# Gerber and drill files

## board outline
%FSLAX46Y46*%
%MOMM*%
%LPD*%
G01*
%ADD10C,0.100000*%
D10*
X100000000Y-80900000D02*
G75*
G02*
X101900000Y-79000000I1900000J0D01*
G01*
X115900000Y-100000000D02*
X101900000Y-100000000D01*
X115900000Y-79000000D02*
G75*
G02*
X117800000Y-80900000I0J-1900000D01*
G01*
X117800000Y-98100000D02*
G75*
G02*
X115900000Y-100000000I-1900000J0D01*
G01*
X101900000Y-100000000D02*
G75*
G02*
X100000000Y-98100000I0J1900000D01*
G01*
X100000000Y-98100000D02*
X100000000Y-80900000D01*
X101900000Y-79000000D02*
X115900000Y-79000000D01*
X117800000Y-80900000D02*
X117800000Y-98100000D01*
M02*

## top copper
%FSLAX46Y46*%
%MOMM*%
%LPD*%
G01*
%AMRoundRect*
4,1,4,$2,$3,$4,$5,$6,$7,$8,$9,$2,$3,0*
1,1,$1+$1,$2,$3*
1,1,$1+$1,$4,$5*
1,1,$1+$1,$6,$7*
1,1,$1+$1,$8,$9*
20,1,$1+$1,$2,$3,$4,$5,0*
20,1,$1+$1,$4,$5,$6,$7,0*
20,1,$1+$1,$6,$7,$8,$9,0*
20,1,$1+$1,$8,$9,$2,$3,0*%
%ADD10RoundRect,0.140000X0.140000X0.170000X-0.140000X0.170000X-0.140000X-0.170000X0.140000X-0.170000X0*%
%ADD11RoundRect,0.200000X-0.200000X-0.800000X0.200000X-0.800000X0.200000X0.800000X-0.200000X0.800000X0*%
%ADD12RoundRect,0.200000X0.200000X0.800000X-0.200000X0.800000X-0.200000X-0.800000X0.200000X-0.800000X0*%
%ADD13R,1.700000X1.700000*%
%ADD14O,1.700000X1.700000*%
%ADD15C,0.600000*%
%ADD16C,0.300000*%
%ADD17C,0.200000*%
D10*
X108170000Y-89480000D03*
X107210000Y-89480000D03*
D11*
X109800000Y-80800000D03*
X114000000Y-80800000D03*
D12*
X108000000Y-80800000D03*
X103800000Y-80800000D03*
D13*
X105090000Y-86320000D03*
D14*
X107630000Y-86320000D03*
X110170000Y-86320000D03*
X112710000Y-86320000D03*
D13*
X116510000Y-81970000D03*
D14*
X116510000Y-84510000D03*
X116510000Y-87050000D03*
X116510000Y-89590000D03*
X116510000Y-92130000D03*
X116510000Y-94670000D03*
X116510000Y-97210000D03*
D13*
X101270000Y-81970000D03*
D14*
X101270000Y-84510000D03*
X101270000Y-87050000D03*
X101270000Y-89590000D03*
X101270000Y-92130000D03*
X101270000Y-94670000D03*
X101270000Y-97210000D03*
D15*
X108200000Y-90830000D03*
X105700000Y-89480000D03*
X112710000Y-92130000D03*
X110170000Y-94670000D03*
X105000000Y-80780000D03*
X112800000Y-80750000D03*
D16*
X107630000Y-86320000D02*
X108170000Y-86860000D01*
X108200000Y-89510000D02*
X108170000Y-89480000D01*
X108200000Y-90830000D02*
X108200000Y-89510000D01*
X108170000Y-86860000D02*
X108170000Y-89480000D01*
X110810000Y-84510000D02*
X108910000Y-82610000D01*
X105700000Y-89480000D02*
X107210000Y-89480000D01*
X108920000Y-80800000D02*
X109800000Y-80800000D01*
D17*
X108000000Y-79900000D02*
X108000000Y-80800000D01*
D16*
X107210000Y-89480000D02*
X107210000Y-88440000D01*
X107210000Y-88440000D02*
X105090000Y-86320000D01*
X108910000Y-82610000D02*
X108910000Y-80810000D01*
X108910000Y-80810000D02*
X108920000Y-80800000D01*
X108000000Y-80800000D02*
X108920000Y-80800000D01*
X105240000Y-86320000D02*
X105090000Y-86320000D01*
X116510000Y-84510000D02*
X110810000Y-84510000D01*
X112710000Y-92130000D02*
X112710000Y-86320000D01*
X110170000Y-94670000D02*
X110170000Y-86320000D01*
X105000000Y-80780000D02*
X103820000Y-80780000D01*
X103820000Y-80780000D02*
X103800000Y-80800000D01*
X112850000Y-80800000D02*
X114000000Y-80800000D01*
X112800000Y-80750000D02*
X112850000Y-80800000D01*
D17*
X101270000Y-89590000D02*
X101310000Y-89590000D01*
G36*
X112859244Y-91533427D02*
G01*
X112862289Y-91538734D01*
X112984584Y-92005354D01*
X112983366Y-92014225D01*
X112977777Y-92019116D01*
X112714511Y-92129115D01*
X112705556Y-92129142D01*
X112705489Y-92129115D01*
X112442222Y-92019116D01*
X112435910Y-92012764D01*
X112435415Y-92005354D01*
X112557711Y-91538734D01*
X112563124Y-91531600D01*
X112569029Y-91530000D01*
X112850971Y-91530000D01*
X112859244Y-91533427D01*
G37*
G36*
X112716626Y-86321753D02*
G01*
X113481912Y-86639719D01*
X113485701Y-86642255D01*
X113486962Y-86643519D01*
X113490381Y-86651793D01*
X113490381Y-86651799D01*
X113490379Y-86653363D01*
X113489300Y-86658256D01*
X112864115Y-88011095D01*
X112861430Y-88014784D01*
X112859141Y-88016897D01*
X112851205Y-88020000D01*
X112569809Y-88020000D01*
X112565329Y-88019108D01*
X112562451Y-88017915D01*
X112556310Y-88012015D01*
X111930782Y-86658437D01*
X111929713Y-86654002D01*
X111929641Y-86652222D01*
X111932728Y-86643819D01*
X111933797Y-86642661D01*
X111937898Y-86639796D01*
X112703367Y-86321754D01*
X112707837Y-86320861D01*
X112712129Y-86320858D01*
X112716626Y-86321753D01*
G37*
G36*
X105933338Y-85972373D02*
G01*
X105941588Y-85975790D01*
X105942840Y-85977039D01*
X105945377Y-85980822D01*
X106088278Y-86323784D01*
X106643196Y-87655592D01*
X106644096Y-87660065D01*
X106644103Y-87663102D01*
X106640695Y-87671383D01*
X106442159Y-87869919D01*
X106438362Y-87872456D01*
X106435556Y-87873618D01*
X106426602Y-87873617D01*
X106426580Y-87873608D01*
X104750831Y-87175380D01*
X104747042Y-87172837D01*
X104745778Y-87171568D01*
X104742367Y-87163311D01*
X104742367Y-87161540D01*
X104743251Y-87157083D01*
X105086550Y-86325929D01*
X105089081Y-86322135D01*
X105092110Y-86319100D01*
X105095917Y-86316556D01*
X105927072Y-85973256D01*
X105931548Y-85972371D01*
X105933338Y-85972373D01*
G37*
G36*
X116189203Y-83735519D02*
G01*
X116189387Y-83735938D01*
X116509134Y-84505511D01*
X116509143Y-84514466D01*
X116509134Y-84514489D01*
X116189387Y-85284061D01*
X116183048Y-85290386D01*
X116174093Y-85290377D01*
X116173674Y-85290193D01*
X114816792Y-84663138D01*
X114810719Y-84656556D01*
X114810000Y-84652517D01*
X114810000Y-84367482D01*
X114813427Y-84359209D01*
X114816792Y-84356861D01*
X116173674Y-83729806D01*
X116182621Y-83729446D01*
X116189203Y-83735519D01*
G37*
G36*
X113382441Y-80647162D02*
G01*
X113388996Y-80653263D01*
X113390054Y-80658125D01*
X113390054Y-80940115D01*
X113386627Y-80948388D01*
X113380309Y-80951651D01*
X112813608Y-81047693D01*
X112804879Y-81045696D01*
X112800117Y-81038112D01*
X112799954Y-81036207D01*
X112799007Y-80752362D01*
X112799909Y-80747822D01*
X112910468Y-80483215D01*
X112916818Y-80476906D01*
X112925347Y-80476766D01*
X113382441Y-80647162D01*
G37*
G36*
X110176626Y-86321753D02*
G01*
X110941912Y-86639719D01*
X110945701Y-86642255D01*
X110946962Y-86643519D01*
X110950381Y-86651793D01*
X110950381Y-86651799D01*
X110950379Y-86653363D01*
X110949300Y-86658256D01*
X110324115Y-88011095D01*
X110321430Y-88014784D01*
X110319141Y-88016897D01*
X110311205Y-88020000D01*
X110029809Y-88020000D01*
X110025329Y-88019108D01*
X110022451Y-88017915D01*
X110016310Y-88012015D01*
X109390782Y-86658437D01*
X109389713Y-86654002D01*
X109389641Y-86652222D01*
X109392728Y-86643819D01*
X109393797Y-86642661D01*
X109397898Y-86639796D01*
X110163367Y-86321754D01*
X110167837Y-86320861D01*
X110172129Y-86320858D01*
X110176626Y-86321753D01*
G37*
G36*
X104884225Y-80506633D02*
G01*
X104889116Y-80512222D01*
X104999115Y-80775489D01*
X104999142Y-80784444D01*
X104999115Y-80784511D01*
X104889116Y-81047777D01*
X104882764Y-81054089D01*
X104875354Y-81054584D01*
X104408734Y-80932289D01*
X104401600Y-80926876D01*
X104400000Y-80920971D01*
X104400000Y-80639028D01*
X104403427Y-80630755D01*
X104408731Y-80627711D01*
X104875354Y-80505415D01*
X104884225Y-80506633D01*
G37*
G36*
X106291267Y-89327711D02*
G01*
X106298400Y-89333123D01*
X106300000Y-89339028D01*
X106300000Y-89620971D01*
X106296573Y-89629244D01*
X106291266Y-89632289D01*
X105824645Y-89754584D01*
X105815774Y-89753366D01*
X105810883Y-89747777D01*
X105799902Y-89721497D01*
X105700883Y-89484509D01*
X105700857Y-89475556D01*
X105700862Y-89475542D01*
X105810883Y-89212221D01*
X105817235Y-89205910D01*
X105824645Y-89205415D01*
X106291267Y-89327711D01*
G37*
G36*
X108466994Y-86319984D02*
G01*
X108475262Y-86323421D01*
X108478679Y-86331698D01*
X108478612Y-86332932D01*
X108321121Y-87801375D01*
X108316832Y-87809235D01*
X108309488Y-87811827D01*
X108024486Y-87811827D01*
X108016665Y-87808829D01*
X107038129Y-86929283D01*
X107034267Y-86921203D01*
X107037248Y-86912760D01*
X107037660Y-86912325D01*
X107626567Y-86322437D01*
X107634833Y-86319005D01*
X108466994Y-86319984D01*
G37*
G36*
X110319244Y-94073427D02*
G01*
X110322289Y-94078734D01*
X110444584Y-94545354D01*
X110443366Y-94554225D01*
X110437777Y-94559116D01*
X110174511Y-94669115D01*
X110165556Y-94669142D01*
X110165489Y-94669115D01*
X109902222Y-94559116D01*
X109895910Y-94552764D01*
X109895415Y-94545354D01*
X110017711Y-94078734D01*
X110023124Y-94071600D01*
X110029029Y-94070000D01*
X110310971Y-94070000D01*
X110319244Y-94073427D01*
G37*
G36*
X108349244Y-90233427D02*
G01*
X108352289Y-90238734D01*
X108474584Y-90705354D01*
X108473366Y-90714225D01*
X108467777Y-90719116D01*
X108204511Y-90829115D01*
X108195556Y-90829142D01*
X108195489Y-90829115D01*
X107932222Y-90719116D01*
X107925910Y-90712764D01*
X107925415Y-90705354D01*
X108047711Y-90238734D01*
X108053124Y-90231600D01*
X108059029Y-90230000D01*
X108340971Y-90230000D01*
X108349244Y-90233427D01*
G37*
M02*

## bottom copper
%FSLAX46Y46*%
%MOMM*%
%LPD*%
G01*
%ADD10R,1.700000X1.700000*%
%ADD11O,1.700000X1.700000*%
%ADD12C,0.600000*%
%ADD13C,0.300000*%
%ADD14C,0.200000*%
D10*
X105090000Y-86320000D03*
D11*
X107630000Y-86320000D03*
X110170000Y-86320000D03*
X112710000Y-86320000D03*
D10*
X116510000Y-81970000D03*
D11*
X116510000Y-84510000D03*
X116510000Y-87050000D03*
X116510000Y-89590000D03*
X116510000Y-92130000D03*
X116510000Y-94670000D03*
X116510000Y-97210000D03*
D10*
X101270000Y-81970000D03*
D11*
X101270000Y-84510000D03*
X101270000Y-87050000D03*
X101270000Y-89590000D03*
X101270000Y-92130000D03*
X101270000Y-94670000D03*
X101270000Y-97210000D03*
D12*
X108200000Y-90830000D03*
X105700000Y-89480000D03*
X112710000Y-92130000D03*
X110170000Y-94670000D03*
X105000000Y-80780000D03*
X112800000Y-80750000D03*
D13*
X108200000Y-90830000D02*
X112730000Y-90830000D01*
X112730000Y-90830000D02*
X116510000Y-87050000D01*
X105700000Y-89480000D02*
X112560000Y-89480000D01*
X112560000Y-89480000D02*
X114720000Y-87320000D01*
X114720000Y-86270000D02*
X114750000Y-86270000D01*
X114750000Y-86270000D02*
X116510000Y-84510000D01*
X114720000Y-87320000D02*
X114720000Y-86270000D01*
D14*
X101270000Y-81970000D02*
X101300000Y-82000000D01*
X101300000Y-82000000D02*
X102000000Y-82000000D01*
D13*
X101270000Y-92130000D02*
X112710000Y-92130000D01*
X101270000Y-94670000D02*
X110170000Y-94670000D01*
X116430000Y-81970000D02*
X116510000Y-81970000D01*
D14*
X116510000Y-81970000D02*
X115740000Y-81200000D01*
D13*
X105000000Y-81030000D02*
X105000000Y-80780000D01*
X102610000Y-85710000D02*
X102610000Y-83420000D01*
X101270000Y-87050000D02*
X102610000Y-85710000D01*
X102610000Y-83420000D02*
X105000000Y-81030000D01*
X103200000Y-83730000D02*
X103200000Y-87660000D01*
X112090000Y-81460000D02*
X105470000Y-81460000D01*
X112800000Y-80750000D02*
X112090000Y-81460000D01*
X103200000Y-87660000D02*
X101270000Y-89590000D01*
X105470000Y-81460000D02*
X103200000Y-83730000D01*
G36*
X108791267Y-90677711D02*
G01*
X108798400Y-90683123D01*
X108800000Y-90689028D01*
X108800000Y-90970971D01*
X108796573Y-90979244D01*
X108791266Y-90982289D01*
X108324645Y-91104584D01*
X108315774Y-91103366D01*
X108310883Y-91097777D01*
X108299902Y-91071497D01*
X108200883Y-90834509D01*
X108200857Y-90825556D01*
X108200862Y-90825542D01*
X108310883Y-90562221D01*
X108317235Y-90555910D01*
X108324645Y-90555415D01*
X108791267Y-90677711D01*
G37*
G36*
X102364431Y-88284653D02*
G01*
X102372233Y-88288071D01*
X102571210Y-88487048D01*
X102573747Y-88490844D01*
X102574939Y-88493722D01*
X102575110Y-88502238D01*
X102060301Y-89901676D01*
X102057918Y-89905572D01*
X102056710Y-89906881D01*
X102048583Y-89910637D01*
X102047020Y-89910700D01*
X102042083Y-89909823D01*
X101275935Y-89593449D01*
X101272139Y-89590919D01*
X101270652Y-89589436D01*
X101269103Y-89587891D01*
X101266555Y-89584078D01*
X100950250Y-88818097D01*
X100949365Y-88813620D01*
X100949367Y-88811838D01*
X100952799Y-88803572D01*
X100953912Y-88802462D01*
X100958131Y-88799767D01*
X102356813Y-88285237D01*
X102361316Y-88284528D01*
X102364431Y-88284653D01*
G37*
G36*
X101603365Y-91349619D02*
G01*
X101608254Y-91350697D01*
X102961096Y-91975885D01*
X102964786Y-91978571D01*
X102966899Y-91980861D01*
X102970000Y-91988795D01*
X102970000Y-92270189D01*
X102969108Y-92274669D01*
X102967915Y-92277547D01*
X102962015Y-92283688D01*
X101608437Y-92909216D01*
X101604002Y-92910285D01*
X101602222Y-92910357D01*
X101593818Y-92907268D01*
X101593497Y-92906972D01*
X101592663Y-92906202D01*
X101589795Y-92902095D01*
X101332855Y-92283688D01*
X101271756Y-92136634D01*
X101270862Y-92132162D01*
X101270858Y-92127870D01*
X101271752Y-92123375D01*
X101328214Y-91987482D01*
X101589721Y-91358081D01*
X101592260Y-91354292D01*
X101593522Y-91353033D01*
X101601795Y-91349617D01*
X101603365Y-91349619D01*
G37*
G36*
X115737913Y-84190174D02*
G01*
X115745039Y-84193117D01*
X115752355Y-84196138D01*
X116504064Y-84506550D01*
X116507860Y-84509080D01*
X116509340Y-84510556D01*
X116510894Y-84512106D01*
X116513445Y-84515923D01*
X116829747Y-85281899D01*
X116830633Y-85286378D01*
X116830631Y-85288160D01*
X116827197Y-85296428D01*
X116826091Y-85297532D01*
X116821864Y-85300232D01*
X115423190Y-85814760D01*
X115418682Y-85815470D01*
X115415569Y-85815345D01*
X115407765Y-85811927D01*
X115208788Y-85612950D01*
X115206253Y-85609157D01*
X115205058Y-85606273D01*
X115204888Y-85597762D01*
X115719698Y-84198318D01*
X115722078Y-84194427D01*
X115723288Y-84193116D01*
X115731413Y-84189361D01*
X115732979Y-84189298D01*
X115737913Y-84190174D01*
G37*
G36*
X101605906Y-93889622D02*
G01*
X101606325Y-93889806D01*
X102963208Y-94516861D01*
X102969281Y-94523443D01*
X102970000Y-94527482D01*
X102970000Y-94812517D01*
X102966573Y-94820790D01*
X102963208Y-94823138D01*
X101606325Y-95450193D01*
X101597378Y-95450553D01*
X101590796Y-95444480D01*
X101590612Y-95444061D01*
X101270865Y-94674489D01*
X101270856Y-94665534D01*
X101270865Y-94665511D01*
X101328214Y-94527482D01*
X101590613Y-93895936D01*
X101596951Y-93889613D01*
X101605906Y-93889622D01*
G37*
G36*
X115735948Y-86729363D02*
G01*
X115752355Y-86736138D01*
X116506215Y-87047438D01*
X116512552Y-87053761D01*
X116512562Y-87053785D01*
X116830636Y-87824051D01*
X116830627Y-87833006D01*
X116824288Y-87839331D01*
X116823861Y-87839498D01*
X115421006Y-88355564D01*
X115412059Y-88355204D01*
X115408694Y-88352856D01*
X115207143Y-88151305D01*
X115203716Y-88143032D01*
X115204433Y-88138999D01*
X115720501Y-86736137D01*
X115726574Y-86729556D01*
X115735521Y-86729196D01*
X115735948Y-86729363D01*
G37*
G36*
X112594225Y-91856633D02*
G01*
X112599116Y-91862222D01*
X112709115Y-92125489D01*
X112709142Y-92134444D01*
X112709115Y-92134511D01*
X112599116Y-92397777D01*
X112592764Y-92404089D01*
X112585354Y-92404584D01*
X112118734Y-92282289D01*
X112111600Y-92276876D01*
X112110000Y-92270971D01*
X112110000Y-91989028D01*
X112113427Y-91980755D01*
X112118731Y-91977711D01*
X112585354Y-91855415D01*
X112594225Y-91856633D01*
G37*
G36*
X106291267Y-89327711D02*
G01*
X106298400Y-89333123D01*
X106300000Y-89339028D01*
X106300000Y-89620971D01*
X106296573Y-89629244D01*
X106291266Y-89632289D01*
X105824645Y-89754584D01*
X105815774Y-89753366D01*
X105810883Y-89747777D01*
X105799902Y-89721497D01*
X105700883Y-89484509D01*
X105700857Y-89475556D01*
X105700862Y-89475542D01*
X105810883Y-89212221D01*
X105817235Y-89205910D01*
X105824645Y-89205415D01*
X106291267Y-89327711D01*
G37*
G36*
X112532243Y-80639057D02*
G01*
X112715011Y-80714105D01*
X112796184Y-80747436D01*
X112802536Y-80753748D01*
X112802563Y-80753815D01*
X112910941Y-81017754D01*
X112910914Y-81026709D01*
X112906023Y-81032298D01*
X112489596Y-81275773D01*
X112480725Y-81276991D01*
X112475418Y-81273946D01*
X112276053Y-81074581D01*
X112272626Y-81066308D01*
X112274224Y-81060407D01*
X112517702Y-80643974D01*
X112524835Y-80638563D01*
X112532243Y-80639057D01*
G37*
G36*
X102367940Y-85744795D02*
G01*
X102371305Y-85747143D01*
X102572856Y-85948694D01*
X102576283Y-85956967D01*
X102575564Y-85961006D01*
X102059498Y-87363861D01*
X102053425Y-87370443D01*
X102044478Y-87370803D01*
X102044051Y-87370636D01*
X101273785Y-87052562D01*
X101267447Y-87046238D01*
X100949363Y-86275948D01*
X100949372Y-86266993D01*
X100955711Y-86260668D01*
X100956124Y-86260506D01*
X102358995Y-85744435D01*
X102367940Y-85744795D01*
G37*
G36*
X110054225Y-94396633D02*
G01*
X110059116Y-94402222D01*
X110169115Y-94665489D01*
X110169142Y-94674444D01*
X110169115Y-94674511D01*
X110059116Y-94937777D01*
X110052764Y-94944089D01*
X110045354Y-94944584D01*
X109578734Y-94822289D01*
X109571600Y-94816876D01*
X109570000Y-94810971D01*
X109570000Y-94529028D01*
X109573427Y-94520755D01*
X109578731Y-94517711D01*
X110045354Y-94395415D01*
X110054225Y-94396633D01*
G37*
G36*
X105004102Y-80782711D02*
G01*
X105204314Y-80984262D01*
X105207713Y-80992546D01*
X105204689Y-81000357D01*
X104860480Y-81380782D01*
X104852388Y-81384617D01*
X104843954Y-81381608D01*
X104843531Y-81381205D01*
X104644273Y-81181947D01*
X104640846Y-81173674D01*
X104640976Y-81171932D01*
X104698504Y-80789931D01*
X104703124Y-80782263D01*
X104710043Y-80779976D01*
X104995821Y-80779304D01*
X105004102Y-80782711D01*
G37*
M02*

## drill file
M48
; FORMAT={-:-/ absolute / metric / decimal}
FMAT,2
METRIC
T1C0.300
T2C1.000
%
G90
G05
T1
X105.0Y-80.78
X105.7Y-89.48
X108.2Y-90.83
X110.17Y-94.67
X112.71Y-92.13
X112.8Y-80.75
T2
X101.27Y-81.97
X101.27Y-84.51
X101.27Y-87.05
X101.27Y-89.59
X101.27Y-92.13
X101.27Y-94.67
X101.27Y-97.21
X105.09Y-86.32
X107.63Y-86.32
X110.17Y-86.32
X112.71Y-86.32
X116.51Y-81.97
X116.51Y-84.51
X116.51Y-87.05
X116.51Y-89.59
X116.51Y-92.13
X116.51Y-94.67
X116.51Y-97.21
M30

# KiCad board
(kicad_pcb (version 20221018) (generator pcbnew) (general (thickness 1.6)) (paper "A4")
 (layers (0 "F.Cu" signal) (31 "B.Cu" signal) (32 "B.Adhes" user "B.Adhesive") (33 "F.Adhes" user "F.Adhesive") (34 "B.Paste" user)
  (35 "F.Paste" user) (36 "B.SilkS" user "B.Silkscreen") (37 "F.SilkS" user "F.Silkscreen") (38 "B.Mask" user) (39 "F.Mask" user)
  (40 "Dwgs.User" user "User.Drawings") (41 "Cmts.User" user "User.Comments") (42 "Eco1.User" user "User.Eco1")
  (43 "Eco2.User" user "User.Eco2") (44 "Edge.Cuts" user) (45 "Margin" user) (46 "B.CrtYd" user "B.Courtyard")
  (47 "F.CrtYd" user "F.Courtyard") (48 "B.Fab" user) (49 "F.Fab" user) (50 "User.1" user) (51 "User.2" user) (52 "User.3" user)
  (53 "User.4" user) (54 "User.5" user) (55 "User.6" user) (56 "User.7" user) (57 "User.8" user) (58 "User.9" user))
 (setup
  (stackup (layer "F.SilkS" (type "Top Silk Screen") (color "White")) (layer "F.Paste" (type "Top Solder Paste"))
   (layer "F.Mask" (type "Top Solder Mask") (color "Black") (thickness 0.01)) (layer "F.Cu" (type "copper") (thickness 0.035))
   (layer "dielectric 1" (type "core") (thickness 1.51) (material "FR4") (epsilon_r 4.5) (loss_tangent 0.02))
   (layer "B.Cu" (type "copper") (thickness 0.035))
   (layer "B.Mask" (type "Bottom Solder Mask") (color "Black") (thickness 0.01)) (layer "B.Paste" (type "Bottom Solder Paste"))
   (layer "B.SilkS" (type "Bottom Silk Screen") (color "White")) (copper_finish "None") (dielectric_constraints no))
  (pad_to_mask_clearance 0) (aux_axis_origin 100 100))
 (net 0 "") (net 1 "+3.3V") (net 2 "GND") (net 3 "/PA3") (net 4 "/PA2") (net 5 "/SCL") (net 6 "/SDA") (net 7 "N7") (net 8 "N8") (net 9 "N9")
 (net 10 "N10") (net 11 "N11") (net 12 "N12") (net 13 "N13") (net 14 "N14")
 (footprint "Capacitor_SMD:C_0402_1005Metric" (layer "F.Cu") (at 107.69 89.48 180)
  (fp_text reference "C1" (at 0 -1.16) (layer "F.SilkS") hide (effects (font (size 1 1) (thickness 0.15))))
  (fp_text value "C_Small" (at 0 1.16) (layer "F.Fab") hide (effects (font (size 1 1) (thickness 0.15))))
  (pad "1" smd roundrect (at -0.48 0 180) (size 0.56 0.62) (layers "F.Cu" "F.Paste" "F.Mask") (roundrect_rratio 0.25) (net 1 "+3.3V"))
  (pad "2" smd roundrect (at 0.48 0 180) (size 0.56 0.62) (layers "F.Cu" "F.Paste" "F.Mask") (roundrect_rratio 0.25) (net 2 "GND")))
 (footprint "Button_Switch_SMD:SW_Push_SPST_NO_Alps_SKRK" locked (layer "F.Cu") (at 111.9 80.8)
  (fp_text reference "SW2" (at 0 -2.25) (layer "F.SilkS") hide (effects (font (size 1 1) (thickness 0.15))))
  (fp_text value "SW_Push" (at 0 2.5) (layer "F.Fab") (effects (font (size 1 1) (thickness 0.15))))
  (pad "1" smd roundrect locked (at -2.1 0) (size 0.8 2) (layers "F.Cu" "F.Paste" "F.Mask") (roundrect_rratio 0.25) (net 2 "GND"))
  (pad "2" smd roundrect locked (at 2.1 0) (size 0.8 2) (layers "F.Cu" "F.Paste" "F.Mask") (roundrect_rratio 0.25) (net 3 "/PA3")))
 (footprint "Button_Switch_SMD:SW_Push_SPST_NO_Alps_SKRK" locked (layer "F.Cu") (at 105.9 80.8 180)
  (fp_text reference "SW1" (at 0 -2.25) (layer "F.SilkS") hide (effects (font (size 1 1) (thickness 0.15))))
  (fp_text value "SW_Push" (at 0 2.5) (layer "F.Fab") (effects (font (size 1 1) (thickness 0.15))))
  (pad "1" smd roundrect locked (at -2.1 0 180) (size 0.8 2) (layers "F.Cu" "F.Paste" "F.Mask") (roundrect_rratio 0.25) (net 2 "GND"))
  (pad "2" smd roundrect locked (at 2.1 0 180) (size 0.8 2) (layers "F.Cu" "F.Paste" "F.Mask") (roundrect_rratio 0.25) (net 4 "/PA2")))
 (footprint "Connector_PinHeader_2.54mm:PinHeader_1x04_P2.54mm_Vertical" (layer "F.Cu") (at 105.09 86.32 90)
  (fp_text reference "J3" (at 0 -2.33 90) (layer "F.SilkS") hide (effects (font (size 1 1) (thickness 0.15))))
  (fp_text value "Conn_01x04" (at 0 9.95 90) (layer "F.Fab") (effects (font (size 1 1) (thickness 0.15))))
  (pad "1" thru_hole rect (at 0 0 90) (size 1.7 1.7) (drill 1) (layers "*.Cu" "*.Mask") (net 2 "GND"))
  (pad "2" thru_hole oval (at 0 2.54 90) (size 1.7 1.7) (drill 1) (layers "*.Cu" "*.Mask") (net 1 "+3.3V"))
  (pad "3" thru_hole oval (at 0 5.08 90) (size 1.7 1.7) (drill 1) (layers "*.Cu" "*.Mask") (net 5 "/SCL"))
  (pad "4" thru_hole oval (at 0 7.62 90) (size 1.7 1.7) (drill 1) (layers "*.Cu" "*.Mask") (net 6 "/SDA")))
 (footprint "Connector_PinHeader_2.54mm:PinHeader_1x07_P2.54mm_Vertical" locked (layer "B.Cu") (at 116.51 81.97 180)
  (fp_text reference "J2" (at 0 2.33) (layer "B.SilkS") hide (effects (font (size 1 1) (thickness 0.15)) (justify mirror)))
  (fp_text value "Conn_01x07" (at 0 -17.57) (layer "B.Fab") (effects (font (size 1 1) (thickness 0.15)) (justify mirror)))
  (pad "1" thru_hole rect locked (at 0 0 180) (size 1.7 1.7) (drill 1) (layers "*.Cu" "*.Mask") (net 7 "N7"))
  (pad "2" thru_hole oval locked (at 0 -2.54 180) (size 1.7 1.7) (drill 1) (layers "*.Cu" "*.Mask") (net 2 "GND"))
  (pad "3" thru_hole oval locked (at 0 -5.08 180) (size 1.7 1.7) (drill 1) (layers "*.Cu" "*.Mask") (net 1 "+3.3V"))
  (pad "4" thru_hole oval locked (at 0 -7.62 180) (size 1.7 1.7) (drill 1) (layers "*.Cu" "*.Mask") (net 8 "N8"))
  (pad "5" thru_hole oval locked (at 0 -10.16 180) (size 1.7 1.7) (drill 1) (layers "*.Cu" "*.Mask") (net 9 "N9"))
  (pad "6" thru_hole oval locked (at 0 -12.7 180) (size 1.7 1.7) (drill 1) (layers "*.Cu" "*.Mask") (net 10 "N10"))
  (pad "7" thru_hole oval locked (at 0 -15.24 180) (size 1.7 1.7) (drill 1) (layers "*.Cu" "*.Mask") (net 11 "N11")))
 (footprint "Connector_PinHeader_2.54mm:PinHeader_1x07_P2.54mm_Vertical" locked (layer "B.Cu") (at 101.27 81.97 180)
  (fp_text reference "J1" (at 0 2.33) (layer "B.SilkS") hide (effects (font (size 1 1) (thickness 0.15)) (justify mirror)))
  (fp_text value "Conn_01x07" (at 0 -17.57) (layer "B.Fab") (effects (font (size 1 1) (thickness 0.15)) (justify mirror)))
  (pad "1" thru_hole rect locked (at 0 0 180) (size 1.7 1.7) (drill 1) (layers "*.Cu" "*.Mask") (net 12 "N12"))
  (pad "2" thru_hole oval locked (at 0 -2.54 180) (size 1.7 1.7) (drill 1) (layers "*.Cu" "*.Mask") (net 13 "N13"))
  (pad "3" thru_hole oval locked (at 0 -5.08 180) (size 1.7 1.7) (drill 1) (layers "*.Cu" "*.Mask") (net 4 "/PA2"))
  (pad "4" thru_hole oval locked (at 0 -7.62 180) (size 1.7 1.7) (drill 1) (layers "*.Cu" "*.Mask") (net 3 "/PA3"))
  (pad "5" thru_hole oval locked (at 0 -10.16 180) (size 1.7 1.7) (drill 1) (layers "*.Cu" "*.Mask") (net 6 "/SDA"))
  (pad "6" thru_hole oval locked (at 0 -12.7 180) (size 1.7 1.7) (drill 1) (layers "*.Cu" "*.Mask") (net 5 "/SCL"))
  (pad "7" thru_hole oval locked (at 0 -15.24 180) (size 1.7 1.7) (drill 1) (layers "*.Cu" "*.Mask") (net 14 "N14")))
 (gr_arc (start 100 80.9) (mid 100.556497 79.556497) (end 101.9 79) (stroke (width 0.1) (type default)) (layer "Edge.Cuts"))
 (gr_line (start 115.9 100) (end 101.9 100) (stroke (width 0.1) (type default)) (layer "Edge.Cuts"))
 (gr_arc (start 115.9 79) (mid 117.243503 79.556497) (end 117.8 80.9) (stroke (width 0.1) (type default)) (layer "Edge.Cuts"))
 (gr_arc (start 117.8 98.1) (mid 117.243503 99.443503) (end 115.9 100) (stroke (width 0.1) (type default)) (layer "Edge.Cuts"))
 (gr_arc (start 101.9 100) (mid 100.556497 99.443503) (end 100 98.1) (stroke (width 0.1) (type default)) (layer "Edge.Cuts"))
 (gr_line (start 100 98.1) (end 100 80.9) (stroke (width 0.1) (type default)) (layer "Edge.Cuts"))
 (gr_line (start 101.9 79) (end 115.9 79) (stroke (width 0.1) (type default)) (layer "Edge.Cuts"))
 (gr_line (start 117.8 80.9) (end 117.8 98.1) (stroke (width 0.1) (type default)) (layer "Edge.Cuts"))
 (segment (start 107.63 86.32) (end 108.17 86.86) (width 0.3) (layer "F.Cu") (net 1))
 (segment (start 108.2 89.51) (end 108.17 89.48) (width 0.3) (layer "F.Cu") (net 1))
 (segment (start 108.2 90.83) (end 108.2 89.51) (width 0.3) (layer "F.Cu") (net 1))
 (segment (start 108.17 86.86) (end 108.17 89.48) (width 0.3) (layer "F.Cu") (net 1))
 (via (at 108.2 90.83) (size 0.6) (drill 0.3) (layers "F.Cu" "B.Cu") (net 1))
 (segment (start 108.2 90.83) (end 112.73 90.83) (width 0.3) (layer "B.Cu") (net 1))
 (segment (start 112.73 90.83) (end 116.51 87.05) (width 0.3) (layer "B.Cu") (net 1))
 (segment (start 110.81 84.51) (end 108.91 82.61) (width 0.3) (layer "F.Cu") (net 2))
 (segment (start 105.7 89.48) (end 107.21 89.48) (width 0.3) (layer "F.Cu") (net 2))
 (segment (start 108.92 80.8) (end 109.8 80.8) (width 0.3) (layer "F.Cu") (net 2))
 (segment (start 108 79.9) (end 108 80.8) (width 0.2) (layer "F.Cu") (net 2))
 (segment (start 107.21 89.48) (end 107.21 88.44) (width 0.3) (layer "F.Cu") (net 2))
 (segment (start 107.21 88.44) (end 105.09 86.32) (width 0.3) (layer "F.Cu") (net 2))
 (segment (start 108.91 82.61) (end 108.91 80.81) (width 0.3) (layer "F.Cu") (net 2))
 (segment (start 108.91 80.81) (end 108.92 80.8) (width 0.3) (layer "F.Cu") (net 2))
 (segment (start 108 80.8) (end 108.92 80.8) (width 0.3) (layer "F.Cu") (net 2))
 (segment (start 105.24 86.32) (end 105.09 86.32) (width 0.3) (layer "F.Cu") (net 2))
 (segment (start 116.51 84.51) (end 110.81 84.51) (width 0.3) (layer "F.Cu") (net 2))
 (via (at 105.7 89.48) (size 0.6) (drill 0.3) (layers "F.Cu" "B.Cu") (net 2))
 (segment (start 105.7 89.48) (end 112.56 89.48) (width 0.3) (layer "B.Cu") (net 2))
 (segment (start 112.56 89.48) (end 114.72 87.32) (width 0.3) (layer "B.Cu") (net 2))
 (segment (start 114.72 86.27) (end 114.75 86.27) (width 0.3) (layer "B.Cu") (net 2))
 (segment (start 114.75 86.27) (end 116.51 84.51) (width 0.3) (layer "B.Cu") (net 2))
 (segment (start 114.72 87.32) (end 114.72 86.27) (width 0.3) (layer "B.Cu") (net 2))
 (segment (start 101.27 81.97) (end 101.3 82) (width 0.2) (layer "B.Cu") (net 12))
 (segment (start 101.3 82) (end 102 82) (width 0.2) (layer "B.Cu") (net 12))
 (segment (start 112.71 92.13) (end 112.71 86.32) (width 0.3) (layer "F.Cu") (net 6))
 (via (at 112.71 92.13) (size 0.6) (drill 0.3) (layers "F.Cu" "B.Cu") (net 6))
 (segment (start 101.27 92.13) (end 112.71 92.13) (width 0.3) (layer "B.Cu") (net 6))
 (segment (start 110.17 94.67) (end 110.17 86.32) (width 0.3) (layer "F.Cu") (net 5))
 (via (at 110.17 94.67) (size 0.6) (drill 0.3) (layers "F.Cu" "B.Cu") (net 5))
 (segment (start 101.27 94.67) (end 110.17 94.67) (width 0.3) (layer "B.Cu") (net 5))
 (segment (start 116.43 81.97) (end 116.51 81.97) (width 0.3) (layer "B.Cu") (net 7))
 (segment (start 116.51 81.97) (end 115.74 81.2) (width 0.2) (layer "B.Cu") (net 7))
 (segment (start 105 80.78) (end 103.82 80.78) (width 0.3) (layer "F.Cu") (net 4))
 (segment (start 103.82 80.78) (end 103.8 80.8) (width 0.3) (layer "F.Cu") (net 4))
 (via (at 105 80.78) (size 0.6) (drill 0.3) (layers "F.Cu" "B.Cu") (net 4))
 (segment (start 105 81.03) (end 105 80.78) (width 0.3) (layer "B.Cu") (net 4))
 (segment (start 102.61 85.71) (end 102.61 83.42) (width 0.3) (layer "B.Cu") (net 4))
 (segment (start 101.27 87.05) (end 102.61 85.71) (width 0.3) (layer "B.Cu") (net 4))
 (segment (start 102.61 83.42) (end 105 81.03) (width 0.3) (layer "B.Cu") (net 4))
 (segment (start 112.85 80.8) (end 114 80.8) (width 0.3) (layer "F.Cu") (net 3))
 (segment (start 112.8 80.75) (end 112.85 80.8) (width 0.3) (layer "F.Cu") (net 3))
 (segment (start 101.27 89.59) (end 101.31 89.59) (width 0.2) (layer "F.Cu") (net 3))
 (via (at 112.8 80.75) (size 0.6) (drill 0.3) (layers "F.Cu" "B.Cu") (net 3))
 (segment (start 103.2 83.73) (end 103.2 87.66) (width 0.3) (layer "B.Cu") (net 3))
 (segment (start 112.09 81.46) (end 105.47 81.46) (width 0.3) (layer "B.Cu") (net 3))
 (segment (start 112.8 80.75) (end 112.09 81.46) (width 0.3) (layer "B.Cu") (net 3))
 (segment (start 103.2 87.66) (end 101.27 89.59) (width 0.3) (layer "B.Cu") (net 3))
 (segment (start 105.47 81.46) (end 103.2 83.73) (width 0.3) (layer "B.Cu") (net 3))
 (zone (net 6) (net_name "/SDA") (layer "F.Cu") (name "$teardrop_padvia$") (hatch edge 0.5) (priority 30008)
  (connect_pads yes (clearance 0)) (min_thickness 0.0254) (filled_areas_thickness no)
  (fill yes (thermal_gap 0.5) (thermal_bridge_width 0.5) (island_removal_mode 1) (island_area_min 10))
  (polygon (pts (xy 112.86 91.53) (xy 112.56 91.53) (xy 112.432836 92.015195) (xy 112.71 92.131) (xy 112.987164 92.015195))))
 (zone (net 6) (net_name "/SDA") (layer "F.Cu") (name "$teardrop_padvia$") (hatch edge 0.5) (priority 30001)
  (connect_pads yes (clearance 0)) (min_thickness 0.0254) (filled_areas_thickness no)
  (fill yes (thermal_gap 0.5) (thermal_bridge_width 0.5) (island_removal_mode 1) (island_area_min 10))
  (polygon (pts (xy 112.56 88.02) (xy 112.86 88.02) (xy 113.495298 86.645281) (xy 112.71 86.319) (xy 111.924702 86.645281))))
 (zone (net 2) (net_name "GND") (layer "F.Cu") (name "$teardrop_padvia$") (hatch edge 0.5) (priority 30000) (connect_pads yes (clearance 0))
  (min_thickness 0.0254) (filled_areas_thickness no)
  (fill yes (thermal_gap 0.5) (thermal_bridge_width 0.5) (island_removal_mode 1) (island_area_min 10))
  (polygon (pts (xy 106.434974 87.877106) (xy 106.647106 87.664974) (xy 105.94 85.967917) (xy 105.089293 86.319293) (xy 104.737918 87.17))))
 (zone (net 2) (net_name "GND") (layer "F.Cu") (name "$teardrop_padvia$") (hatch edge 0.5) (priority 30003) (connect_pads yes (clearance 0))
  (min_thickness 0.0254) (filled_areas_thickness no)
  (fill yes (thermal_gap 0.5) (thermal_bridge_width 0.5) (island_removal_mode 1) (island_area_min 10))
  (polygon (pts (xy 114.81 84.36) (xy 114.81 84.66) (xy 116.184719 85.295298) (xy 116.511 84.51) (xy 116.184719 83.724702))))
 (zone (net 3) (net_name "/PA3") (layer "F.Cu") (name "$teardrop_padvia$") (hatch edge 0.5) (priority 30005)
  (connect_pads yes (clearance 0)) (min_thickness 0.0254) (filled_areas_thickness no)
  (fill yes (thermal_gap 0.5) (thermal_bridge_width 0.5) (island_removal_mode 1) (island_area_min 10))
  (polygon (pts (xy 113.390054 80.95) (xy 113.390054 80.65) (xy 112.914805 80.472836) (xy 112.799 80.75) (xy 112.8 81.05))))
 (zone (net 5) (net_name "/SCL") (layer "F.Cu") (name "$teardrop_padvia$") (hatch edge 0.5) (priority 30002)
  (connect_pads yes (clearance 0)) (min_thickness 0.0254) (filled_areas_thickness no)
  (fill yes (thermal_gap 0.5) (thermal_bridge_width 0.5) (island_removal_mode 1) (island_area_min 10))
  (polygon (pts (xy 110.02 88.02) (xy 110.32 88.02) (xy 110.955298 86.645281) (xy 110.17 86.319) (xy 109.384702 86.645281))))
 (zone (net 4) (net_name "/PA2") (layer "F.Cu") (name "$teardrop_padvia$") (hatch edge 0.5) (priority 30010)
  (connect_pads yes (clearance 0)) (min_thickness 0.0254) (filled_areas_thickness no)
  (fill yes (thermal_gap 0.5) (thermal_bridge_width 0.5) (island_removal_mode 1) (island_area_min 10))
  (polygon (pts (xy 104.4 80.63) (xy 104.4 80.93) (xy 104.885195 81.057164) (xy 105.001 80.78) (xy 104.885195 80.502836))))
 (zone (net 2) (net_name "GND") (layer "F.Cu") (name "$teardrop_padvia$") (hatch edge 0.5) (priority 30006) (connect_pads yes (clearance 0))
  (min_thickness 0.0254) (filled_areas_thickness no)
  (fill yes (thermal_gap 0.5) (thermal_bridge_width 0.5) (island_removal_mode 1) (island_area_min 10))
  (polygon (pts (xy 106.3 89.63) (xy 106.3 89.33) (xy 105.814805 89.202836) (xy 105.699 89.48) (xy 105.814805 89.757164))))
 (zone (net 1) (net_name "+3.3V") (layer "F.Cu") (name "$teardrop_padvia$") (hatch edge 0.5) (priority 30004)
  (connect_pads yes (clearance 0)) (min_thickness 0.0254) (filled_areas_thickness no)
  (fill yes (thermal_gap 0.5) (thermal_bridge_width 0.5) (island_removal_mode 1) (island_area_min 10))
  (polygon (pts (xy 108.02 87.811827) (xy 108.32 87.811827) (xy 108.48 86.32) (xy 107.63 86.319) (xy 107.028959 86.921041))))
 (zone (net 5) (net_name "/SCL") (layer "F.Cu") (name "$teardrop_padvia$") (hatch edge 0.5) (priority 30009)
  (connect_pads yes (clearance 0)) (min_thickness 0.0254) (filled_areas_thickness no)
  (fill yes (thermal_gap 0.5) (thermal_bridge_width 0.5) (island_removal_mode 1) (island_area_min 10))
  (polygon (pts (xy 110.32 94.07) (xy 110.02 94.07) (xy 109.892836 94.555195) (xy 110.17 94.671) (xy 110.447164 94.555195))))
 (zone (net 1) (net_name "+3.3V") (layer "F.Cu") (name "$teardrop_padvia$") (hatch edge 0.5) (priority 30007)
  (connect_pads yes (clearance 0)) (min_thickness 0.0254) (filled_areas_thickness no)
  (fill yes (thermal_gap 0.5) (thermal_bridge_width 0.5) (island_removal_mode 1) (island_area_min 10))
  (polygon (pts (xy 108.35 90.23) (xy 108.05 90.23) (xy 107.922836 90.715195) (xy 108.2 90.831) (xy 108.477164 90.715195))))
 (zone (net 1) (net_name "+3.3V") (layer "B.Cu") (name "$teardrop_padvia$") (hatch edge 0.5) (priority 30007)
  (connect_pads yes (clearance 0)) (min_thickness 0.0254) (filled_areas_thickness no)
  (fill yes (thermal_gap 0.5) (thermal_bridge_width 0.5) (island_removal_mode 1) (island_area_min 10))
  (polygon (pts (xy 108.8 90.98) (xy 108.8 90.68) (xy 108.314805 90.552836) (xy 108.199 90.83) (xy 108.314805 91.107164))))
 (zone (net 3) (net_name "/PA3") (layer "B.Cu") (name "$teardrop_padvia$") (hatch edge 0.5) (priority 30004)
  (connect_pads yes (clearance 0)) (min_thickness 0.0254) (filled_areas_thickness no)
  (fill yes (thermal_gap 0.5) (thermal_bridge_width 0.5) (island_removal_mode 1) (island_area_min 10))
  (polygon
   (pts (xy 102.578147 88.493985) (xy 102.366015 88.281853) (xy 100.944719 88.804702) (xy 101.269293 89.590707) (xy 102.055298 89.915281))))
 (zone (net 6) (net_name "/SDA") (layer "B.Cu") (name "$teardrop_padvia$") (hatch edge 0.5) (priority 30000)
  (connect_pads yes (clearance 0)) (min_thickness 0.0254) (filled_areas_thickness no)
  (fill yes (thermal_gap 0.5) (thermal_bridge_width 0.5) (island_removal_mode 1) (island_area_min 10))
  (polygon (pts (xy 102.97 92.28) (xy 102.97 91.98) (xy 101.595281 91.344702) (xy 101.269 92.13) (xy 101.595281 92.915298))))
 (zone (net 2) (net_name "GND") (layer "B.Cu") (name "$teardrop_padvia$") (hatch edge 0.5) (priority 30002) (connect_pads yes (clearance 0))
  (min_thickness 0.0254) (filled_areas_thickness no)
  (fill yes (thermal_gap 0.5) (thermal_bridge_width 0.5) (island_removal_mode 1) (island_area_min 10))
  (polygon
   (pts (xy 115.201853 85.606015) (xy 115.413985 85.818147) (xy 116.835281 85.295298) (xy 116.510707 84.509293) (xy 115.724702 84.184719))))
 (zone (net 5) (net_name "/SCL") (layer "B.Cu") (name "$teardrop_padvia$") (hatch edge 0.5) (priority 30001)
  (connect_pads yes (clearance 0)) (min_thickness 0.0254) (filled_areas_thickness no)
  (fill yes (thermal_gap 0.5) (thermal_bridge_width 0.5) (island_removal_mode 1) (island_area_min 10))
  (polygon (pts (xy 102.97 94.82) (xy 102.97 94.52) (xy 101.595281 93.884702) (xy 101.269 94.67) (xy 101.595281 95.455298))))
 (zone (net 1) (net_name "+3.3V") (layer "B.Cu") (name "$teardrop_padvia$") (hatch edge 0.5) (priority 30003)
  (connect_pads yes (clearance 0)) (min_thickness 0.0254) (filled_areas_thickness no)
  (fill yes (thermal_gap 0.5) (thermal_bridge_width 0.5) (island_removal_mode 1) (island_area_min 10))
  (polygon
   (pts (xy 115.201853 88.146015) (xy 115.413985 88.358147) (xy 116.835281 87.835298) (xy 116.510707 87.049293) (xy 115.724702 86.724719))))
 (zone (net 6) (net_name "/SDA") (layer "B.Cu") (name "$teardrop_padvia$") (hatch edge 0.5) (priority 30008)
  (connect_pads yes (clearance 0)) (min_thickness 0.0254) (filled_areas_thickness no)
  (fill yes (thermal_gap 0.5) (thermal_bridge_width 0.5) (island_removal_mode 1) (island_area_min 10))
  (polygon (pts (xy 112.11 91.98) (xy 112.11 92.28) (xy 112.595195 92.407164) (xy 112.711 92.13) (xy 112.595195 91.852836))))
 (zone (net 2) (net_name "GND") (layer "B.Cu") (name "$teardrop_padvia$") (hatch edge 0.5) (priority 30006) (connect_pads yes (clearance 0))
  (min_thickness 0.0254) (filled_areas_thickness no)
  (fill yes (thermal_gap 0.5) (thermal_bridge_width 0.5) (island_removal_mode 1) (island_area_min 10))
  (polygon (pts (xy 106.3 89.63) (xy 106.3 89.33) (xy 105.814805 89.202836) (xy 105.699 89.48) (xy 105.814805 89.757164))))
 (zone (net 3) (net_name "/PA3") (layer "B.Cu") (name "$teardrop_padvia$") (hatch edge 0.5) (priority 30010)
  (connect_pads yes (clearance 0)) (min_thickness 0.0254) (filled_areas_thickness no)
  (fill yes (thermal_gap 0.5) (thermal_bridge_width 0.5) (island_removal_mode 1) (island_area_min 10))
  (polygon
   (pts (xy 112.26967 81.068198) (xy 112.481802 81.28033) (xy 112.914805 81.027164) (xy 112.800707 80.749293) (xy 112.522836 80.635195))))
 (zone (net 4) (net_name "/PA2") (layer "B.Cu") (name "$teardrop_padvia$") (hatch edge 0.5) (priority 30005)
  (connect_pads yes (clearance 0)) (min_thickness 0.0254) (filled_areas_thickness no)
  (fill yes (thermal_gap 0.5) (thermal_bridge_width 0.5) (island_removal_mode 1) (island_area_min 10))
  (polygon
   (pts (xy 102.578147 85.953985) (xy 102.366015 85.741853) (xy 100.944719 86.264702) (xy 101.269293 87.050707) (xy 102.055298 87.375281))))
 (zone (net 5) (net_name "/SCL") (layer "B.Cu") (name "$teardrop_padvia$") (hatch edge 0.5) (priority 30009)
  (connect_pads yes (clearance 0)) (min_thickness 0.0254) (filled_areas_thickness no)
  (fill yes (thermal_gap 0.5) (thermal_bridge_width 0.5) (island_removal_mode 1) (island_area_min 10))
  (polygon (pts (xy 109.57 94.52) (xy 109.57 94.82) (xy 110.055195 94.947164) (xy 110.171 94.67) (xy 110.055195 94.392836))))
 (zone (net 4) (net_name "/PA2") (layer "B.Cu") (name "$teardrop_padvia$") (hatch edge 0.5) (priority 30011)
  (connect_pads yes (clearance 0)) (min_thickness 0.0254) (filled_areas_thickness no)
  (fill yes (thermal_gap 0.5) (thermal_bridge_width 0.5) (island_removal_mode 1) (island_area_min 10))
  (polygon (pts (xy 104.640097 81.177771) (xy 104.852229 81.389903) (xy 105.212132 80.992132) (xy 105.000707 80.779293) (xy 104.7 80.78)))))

